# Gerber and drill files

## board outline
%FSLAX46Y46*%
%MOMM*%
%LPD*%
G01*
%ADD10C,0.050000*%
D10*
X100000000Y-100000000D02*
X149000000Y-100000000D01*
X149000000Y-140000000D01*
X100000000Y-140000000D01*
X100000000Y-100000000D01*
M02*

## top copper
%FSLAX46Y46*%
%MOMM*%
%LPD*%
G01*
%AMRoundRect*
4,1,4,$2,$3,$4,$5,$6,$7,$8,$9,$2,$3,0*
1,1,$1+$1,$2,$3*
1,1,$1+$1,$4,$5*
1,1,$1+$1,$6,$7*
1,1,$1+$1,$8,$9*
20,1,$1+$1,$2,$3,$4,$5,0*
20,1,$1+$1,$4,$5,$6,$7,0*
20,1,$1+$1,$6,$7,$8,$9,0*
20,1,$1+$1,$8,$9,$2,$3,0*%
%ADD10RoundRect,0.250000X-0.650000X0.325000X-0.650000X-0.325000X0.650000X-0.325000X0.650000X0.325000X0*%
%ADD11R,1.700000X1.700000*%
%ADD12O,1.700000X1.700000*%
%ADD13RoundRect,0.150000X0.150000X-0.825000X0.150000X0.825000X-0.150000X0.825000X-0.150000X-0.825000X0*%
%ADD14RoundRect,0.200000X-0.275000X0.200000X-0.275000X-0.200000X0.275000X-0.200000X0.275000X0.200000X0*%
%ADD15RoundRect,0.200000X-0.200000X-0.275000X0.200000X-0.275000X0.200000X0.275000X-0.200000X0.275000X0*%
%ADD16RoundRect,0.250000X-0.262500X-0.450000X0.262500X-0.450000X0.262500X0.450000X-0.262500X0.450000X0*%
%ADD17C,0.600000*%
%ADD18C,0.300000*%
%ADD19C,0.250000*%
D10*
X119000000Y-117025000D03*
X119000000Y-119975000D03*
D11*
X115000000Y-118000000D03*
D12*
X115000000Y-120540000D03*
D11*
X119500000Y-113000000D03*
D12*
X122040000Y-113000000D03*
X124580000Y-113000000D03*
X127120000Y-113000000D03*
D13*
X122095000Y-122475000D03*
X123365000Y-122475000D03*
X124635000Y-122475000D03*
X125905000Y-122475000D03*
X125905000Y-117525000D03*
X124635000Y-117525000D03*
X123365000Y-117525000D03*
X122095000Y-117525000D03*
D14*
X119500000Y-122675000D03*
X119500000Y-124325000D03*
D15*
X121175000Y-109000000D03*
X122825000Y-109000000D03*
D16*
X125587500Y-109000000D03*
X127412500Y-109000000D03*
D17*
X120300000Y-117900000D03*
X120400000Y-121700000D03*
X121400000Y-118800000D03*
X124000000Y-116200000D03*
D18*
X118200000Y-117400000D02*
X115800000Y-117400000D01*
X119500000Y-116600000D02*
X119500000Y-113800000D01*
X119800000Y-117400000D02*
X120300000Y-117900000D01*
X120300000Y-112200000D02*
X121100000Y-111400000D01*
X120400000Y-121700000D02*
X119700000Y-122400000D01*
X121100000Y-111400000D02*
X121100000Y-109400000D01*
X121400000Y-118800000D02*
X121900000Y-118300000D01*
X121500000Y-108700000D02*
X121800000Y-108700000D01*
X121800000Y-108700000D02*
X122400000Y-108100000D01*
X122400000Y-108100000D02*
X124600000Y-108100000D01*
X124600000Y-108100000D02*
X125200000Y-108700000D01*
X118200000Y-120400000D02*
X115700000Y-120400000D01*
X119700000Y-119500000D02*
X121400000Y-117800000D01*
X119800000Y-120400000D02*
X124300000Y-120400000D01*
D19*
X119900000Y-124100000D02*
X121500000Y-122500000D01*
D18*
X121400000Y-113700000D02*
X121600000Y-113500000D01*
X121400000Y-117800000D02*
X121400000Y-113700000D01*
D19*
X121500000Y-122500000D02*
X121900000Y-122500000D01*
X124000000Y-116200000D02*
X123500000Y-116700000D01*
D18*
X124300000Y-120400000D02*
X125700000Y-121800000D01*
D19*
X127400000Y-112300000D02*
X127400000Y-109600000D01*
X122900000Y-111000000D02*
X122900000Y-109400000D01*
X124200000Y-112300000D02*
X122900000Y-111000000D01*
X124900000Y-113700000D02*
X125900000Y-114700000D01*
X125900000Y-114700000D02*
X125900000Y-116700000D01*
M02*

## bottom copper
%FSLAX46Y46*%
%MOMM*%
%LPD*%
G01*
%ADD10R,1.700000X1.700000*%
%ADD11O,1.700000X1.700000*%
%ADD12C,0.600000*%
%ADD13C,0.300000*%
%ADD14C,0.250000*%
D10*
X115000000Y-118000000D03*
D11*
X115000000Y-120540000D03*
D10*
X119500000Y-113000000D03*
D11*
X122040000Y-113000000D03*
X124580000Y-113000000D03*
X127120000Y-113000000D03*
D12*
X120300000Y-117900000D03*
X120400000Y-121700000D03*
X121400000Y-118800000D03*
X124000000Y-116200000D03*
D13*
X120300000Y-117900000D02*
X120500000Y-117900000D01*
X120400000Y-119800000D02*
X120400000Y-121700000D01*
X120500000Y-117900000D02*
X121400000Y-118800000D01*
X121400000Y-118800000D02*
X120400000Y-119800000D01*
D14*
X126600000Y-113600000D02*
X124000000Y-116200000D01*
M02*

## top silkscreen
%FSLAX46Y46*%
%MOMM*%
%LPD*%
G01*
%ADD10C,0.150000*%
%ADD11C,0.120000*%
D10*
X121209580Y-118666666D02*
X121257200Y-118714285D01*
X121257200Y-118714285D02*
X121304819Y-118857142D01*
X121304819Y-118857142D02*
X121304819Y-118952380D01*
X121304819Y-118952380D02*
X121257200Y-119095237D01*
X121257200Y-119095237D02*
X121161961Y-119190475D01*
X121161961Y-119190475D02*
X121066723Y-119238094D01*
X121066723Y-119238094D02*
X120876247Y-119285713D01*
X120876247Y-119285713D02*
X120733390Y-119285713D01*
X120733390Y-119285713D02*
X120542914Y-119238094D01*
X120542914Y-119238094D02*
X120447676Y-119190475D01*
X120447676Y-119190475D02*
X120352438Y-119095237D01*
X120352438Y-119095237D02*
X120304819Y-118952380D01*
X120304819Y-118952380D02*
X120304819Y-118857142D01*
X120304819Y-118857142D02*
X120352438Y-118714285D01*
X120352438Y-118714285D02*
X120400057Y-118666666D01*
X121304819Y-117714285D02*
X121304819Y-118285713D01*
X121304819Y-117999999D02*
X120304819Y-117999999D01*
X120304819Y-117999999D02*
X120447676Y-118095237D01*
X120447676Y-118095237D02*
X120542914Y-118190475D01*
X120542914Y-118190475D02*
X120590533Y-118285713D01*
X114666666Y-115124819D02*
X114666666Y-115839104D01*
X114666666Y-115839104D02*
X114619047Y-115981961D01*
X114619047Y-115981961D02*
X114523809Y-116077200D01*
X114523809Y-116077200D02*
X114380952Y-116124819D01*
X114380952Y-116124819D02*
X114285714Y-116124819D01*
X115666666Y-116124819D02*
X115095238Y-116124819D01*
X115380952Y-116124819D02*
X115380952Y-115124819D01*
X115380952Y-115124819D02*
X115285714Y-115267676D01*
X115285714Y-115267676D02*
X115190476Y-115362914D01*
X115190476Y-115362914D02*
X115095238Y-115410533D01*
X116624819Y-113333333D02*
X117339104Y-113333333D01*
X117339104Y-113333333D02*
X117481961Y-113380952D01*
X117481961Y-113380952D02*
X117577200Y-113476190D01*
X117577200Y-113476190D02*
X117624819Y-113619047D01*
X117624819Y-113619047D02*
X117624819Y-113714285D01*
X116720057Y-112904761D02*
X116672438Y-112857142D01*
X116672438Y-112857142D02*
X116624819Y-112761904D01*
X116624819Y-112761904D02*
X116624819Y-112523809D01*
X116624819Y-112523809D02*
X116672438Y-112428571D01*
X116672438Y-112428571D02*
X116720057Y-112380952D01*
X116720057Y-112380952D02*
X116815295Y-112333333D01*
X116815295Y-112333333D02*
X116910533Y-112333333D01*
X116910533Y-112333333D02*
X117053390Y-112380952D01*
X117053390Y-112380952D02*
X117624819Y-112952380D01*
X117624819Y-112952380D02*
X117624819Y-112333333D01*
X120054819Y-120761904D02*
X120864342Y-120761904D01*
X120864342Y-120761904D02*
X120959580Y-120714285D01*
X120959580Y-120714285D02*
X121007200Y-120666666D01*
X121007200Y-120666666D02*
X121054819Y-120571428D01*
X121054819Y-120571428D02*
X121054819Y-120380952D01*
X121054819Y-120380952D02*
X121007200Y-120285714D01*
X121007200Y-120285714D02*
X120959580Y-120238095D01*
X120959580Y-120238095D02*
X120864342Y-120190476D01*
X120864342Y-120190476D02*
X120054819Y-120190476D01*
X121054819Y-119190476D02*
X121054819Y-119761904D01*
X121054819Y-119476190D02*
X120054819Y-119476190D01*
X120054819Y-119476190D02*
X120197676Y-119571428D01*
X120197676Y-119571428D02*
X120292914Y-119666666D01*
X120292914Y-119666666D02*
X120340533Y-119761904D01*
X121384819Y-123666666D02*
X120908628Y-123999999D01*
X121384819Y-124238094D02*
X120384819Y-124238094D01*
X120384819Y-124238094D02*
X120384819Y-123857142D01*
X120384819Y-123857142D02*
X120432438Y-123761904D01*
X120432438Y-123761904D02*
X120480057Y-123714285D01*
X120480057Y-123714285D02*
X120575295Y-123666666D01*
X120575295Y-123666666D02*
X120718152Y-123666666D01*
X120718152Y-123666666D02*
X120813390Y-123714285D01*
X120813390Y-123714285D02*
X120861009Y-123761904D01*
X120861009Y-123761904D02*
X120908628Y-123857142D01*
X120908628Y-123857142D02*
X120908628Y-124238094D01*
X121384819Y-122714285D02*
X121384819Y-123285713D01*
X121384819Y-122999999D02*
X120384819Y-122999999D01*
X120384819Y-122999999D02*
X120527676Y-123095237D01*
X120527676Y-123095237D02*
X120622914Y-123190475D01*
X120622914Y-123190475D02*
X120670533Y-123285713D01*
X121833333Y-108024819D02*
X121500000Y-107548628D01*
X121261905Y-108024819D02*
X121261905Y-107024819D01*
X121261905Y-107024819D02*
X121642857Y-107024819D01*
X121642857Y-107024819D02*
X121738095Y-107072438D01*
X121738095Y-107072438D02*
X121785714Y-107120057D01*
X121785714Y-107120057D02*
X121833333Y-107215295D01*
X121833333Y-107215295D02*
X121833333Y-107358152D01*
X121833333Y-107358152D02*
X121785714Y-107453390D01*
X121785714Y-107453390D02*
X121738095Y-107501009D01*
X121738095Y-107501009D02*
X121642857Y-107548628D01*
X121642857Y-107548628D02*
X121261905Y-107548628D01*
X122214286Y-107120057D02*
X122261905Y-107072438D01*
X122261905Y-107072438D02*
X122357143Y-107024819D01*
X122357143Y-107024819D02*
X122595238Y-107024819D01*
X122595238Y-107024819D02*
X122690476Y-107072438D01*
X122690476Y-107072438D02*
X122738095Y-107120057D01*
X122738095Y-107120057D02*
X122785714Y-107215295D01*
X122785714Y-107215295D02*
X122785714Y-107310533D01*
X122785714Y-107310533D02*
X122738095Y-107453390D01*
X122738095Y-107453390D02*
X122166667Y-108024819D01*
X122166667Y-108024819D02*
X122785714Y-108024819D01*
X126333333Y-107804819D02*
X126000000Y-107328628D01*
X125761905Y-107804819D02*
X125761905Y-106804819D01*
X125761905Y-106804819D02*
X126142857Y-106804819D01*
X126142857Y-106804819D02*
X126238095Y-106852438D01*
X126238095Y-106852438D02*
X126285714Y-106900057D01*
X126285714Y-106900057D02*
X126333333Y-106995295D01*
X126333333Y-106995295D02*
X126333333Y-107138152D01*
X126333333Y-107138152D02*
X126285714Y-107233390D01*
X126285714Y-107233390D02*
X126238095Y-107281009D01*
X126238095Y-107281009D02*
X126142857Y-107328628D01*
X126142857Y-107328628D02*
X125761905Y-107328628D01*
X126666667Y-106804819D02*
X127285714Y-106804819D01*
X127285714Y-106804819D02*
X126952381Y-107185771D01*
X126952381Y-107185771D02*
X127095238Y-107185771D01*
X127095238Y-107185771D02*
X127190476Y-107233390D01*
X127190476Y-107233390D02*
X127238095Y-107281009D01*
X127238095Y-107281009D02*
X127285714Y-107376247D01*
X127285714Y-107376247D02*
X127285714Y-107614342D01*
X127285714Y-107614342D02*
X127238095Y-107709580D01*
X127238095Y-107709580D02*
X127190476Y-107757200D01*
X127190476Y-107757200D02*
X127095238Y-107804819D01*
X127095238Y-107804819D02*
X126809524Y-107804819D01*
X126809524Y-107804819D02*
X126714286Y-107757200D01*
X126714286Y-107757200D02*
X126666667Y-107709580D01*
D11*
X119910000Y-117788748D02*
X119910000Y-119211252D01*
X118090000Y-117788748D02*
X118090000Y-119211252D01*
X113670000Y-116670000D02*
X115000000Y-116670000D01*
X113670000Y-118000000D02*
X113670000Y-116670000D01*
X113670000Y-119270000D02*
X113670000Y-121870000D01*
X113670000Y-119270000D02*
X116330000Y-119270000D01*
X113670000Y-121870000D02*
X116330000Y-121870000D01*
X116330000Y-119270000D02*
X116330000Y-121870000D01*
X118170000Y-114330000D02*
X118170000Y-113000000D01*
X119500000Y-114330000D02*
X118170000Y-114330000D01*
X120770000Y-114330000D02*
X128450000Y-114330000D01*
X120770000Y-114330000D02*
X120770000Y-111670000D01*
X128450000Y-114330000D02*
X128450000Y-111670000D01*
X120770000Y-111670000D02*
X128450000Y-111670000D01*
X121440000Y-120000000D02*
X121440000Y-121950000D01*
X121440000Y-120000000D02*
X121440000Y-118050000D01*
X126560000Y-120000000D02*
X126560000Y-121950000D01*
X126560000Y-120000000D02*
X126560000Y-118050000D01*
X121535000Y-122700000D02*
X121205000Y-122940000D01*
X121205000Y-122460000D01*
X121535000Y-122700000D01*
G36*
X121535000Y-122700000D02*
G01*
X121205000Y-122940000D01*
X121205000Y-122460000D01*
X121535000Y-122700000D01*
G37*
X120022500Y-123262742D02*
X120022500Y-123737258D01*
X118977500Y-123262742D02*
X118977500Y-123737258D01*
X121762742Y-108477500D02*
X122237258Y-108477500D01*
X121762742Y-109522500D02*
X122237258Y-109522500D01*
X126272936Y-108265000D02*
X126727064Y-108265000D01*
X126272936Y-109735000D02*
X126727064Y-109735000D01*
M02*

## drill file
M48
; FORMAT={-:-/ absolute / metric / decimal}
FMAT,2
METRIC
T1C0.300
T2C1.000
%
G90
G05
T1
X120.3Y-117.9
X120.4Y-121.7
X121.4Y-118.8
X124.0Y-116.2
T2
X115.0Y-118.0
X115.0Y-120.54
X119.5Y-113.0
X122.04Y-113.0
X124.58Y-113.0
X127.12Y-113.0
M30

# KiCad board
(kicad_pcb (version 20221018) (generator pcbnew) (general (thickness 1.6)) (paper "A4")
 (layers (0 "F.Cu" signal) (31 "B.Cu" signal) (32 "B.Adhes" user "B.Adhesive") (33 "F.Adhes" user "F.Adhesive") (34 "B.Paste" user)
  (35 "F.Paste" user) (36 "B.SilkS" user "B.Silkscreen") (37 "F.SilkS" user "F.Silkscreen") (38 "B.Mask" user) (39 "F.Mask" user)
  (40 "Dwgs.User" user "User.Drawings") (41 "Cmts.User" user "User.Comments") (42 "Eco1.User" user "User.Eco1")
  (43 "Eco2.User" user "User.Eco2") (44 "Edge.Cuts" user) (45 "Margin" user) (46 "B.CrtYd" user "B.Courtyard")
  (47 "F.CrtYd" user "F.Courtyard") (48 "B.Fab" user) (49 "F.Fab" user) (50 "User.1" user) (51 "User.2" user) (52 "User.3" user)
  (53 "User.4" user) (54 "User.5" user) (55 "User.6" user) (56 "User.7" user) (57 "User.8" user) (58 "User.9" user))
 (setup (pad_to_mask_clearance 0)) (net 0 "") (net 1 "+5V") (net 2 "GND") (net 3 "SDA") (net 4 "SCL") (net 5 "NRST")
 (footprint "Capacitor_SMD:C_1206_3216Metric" (layer "F.Cu") (at 119 118.5 -90)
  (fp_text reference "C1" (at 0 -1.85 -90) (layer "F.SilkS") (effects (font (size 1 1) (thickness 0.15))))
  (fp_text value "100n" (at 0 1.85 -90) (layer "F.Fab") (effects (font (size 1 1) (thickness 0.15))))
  (fp_line (start -0.711252 -0.91) (end 0.711252 -0.91) (stroke (width 0.12) (type solid)) (layer "F.SilkS"))
  (fp_line (start -0.711252 0.91) (end 0.711252 0.91) (stroke (width 0.12) (type solid)) (layer "F.SilkS"))
  (pad "1" smd roundrect (at -1.475 0 270) (size 1.15 1.8) (layers "F.Cu" "F.Paste" "F.Mask") (roundrect_rratio 0.217391) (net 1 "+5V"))
  (pad "2" smd roundrect (at 1.475 0 270) (size 1.15 1.8) (layers "F.Cu" "F.Paste" "F.Mask") (roundrect_rratio 0.217391) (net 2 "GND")))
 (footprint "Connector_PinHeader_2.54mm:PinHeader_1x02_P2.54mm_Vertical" (layer "F.Cu") (at 115 118)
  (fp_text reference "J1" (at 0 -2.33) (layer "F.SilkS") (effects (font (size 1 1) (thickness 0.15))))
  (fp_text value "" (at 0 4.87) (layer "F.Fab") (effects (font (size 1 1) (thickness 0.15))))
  (fp_line (start -1.33 -1.33) (end 0 -1.33) (stroke (width 0.12) (type solid)) (layer "F.SilkS"))
  (fp_line (start -1.33 0) (end -1.33 -1.33) (stroke (width 0.12) (type solid)) (layer "F.SilkS"))
  (fp_line (start -1.33 1.27) (end -1.33 3.87) (stroke (width 0.12) (type solid)) (layer "F.SilkS"))
  (fp_line (start -1.33 1.27) (end 1.33 1.27) (stroke (width 0.12) (type solid)) (layer "F.SilkS"))
  (fp_line (start -1.33 3.87) (end 1.33 3.87) (stroke (width 0.12) (type solid)) (layer "F.SilkS"))
  (fp_line (start 1.33 1.27) (end 1.33 3.87) (stroke (width 0.12) (type solid)) (layer "F.SilkS"))
  (pad "1" thru_hole rect (at 0 0) (size 1.7 1.7) (drill 1) (layers "*.Cu" "*.Mask") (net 1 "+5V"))
  (pad "2" thru_hole oval (at 0 2.54) (size 1.7 1.7) (drill 1) (layers "*.Cu" "*.Mask") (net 2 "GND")))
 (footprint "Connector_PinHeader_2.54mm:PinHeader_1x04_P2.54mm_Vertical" (layer "F.Cu") (at 119.5 113 90)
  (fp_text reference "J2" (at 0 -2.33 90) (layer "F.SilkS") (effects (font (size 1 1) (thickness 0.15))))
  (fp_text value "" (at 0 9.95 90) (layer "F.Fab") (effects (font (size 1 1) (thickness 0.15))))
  (fp_line (start -1.33 -1.33) (end 0 -1.33) (stroke (width 0.12) (type solid)) (layer "F.SilkS"))
  (fp_line (start -1.33 0) (end -1.33 -1.33) (stroke (width 0.12) (type solid)) (layer "F.SilkS"))
  (fp_line (start -1.33 1.27) (end -1.33 8.95) (stroke (width 0.12) (type solid)) (layer "F.SilkS"))
  (fp_line (start -1.33 1.27) (end 1.33 1.27) (stroke (width 0.12) (type solid)) (layer "F.SilkS"))
  (fp_line (start -1.33 8.95) (end 1.33 8.95) (stroke (width 0.12) (type solid)) (layer "F.SilkS"))
  (fp_line (start 1.33 1.27) (end 1.33 8.95) (stroke (width 0.12) (type solid)) (layer "F.SilkS"))
  (pad "1" thru_hole rect (at 0 0 90) (size 1.7 1.7) (drill 1) (layers "*.Cu" "*.Mask") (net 1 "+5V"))
  (pad "2" thru_hole oval (at 0 2.54 90) (size 1.7 1.7) (drill 1) (layers "*.Cu" "*.Mask") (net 2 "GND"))
  (pad "3" thru_hole oval (at 0 5.08 90) (size 1.7 1.7) (drill 1) (layers "*.Cu" "*.Mask") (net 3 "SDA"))
  (pad "4" thru_hole oval (at 0 7.62 90) (size 1.7 1.7) (drill 1) (layers "*.Cu" "*.Mask") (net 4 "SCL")))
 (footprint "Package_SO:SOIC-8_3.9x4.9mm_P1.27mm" (layer "F.Cu") (at 124 120 90)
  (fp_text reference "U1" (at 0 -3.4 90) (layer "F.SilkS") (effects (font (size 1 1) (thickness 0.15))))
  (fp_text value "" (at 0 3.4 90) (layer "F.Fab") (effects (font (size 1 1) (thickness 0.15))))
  (fp_line (start 0 -2.56) (end -1.95 -2.56) (stroke (width 0.12) (type solid)) (layer "F.SilkS"))
  (fp_line (start 0 -2.56) (end 1.95 -2.56) (stroke (width 0.12) (type solid)) (layer "F.SilkS"))
  (fp_line (start 0 2.56) (end -1.95 2.56) (stroke (width 0.12) (type solid)) (layer "F.SilkS"))
  (fp_line (start 0 2.56) (end 1.95 2.56) (stroke (width 0.12) (type solid)) (layer "F.SilkS"))
  (fp_poly
   (pts (xy -2.7 -2.465) (xy -2.94 -2.795) (xy -2.46 -2.795) (xy -2.7 -2.465)) (stroke (width 0.12) (type solid)) (fill solid)
   (layer "F.SilkS"))
  (pad "1" smd roundrect (at -2.475 -1.905 90) (size 1.95 0.6) (layers "F.Cu" "F.Paste" "F.Mask") (roundrect_rratio 0.25) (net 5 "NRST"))
  (pad "2" smd roundrect (at -2.475 -0.635 90) (size 1.95 0.6) (layers "F.Cu" "F.Paste" "F.Mask") (roundrect_rratio 0.25))
  (pad "3" smd roundrect (at -2.475 0.635 90) (size 1.95 0.6) (layers "F.Cu" "F.Paste" "F.Mask") (roundrect_rratio 0.25))
  (pad "4" smd roundrect (at -2.475 1.905 90) (size 1.95 0.6) (layers "F.Cu" "F.Paste" "F.Mask") (roundrect_rratio 0.25) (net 2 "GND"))
  (pad "5" smd roundrect (at 2.475 1.905 90) (size 1.95 0.6) (layers "F.Cu" "F.Paste" "F.Mask") (roundrect_rratio 0.25) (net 3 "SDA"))
  (pad "6" smd roundrect (at 2.475 0.635 90) (size 1.95 0.6) (layers "F.Cu" "F.Paste" "F.Mask") (roundrect_rratio 0.25))
  (pad "7" smd roundrect (at 2.475 -0.635 90) (size 1.95 0.6) (layers "F.Cu" "F.Paste" "F.Mask") (roundrect_rratio 0.25) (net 4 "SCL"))
  (pad "8" smd roundrect (at 2.475 -1.905 90) (size 1.95 0.6) (layers "F.Cu" "F.Paste" "F.Mask") (roundrect_rratio 0.25) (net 1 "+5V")))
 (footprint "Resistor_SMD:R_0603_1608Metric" (layer "F.Cu") (at 119.5 123.5 -90)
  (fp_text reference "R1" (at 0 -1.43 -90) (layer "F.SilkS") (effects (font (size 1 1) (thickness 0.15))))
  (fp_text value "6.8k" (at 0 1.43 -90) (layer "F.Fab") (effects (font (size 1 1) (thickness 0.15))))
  (fp_line (start -0.237258 -0.5225) (end 0.237258 -0.5225) (stroke (width 0.12) (type solid)) (layer "F.SilkS"))
  (fp_line (start -0.237258 0.5225) (end 0.237258 0.5225) (stroke (width 0.12) (type solid)) (layer "F.SilkS"))
  (pad "1" smd roundrect (at -0.825 0 270) (size 0.8 0.95) (layers "F.Cu" "F.Paste" "F.Mask") (roundrect_rratio 0.25) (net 1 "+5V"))
  (pad "2" smd roundrect (at 0.825 0 270) (size 0.8 0.95) (layers "F.Cu" "F.Paste" "F.Mask") (roundrect_rratio 0.25) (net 5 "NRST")))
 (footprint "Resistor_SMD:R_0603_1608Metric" (layer "F.Cu") (at 122 109)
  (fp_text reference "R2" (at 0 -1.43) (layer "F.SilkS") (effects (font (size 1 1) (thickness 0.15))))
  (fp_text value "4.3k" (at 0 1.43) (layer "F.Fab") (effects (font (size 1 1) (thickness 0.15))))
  (fp_line (start -0.237258 -0.5225) (end 0.237258 -0.5225) (stroke (width 0.12) (type solid)) (layer "F.SilkS"))
  (fp_line (start -0.237258 0.5225) (end 0.237258 0.5225) (stroke (width 0.12) (type solid)) (layer "F.SilkS"))
  (pad "1" smd roundrect (at -0.825 0) (size 0.8 0.95) (layers "F.Cu" "F.Paste" "F.Mask") (roundrect_rratio 0.25) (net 1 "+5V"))
  (pad "2" smd roundrect (at 0.825 0) (size 0.8 0.95) (layers "F.Cu" "F.Paste" "F.Mask") (roundrect_rratio 0.25) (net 3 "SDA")))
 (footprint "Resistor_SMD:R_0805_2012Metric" (layer "F.Cu") (at 126.5 109)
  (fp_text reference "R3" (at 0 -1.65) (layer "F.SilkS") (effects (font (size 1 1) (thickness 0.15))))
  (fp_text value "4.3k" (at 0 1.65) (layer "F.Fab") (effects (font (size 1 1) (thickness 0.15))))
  (fp_line (start -0.227064 -0.735) (end 0.227064 -0.735) (stroke (width 0.12) (type solid)) (layer "F.SilkS"))
  (fp_line (start -0.227064 0.735) (end 0.227064 0.735) (stroke (width 0.12) (type solid)) (layer "F.SilkS"))
  (pad "1" smd roundrect (at -0.9125 0) (size 1.025 1.4) (layers "F.Cu" "F.Paste" "F.Mask") (roundrect_rratio 0.243902) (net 1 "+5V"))
  (pad "2" smd roundrect (at 0.9125 0) (size 1.025 1.4) (layers "F.Cu" "F.Paste" "F.Mask") (roundrect_rratio 0.243902) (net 4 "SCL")))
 (gr_rect (start 100 100) (end 149 140) (stroke (width 0.05) (type default)) (fill none) (layer "Edge.Cuts"))
 (segment (start 118.2 117.4) (end 115.8 117.4) (width 0.3) (layer "F.Cu") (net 1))
 (segment (start 119.5 116.6) (end 119.5 113.8) (width 0.3) (layer "F.Cu") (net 1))
 (segment (start 119.8 117.4) (end 120.3 117.9) (width 0.3) (layer "F.Cu") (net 1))
 (segment (start 120.3 112.2) (end 121.1 111.4) (width 0.3) (layer "F.Cu") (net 1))
 (segment (start 120.4 121.7) (end 119.7 122.4) (width 0.3) (layer "F.Cu") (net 1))
 (segment (start 121.1 111.4) (end 121.1 109.4) (width 0.3) (layer "F.Cu") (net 1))
 (segment (start 121.4 118.8) (end 121.9 118.3) (width 0.3) (layer "F.Cu") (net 1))
 (segment (start 121.5 108.7) (end 121.8 108.7) (width 0.3) (layer "F.Cu") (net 1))
 (segment (start 121.8 108.7) (end 122.4 108.1) (width 0.3) (layer "F.Cu") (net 1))
 (segment (start 122.4 108.1) (end 124.6 108.1) (width 0.3) (layer "F.Cu") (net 1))
 (segment (start 124.6 108.1) (end 125.2 108.7) (width 0.3) (layer "F.Cu") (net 1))
 (via (at 120.3 117.9) (size 0.6) (drill 0.3) (layers "F.Cu" "B.Cu") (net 1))
 (via (at 120.4 121.7) (size 0.6) (drill 0.3) (layers "F.Cu" "B.Cu") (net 1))
 (via (at 121.4 118.8) (size 0.6) (drill 0.3) (layers "F.Cu" "B.Cu") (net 1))
 (segment (start 118.2 120.4) (end 115.7 120.4) (width 0.3) (layer "F.Cu") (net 2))
 (segment (start 119.7 119.5) (end 121.4 117.8) (width 0.3) (layer "F.Cu") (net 2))
 (segment (start 119.8 120.4) (end 124.3 120.4) (width 0.3) (layer "F.Cu") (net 2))
 (segment (start 119.9 124.1) (end 121.5 122.5) (width 0.25) (layer "F.Cu") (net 5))
 (segment (start 120.3 117.9) (end 120.5 117.9) (width 0.3) (layer "B.Cu") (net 1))
 (segment (start 120.4 119.8) (end 120.4 121.7) (width 0.3) (layer "B.Cu") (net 1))
 (segment (start 120.5 117.9) (end 121.4 118.8) (width 0.3) (layer "B.Cu") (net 1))
 (segment (start 121.4 113.7) (end 121.6 113.5) (width 0.3) (layer "F.Cu") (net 2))
 (segment (start 121.4 117.8) (end 121.4 113.7) (width 0.3) (layer "F.Cu") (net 2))
 (segment (start 121.4 118.8) (end 120.4 119.8) (width 0.3) (layer "B.Cu") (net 1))
 (segment (start 121.5 122.5) (end 121.9 122.5) (width 0.25) (layer "F.Cu") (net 5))
 (segment (start 124 116.2) (end 123.5 116.7) (width 0.25) (layer "F.Cu") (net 4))
 (segment (start 124.3 120.4) (end 125.7 121.8) (width 0.3) (layer "F.Cu") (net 2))
 (segment (start 127.4 112.3) (end 127.4 109.6) (width 0.25) (layer "F.Cu") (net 4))
 (via (at 124 116.2) (size 0.6) (drill 0.3) (layers "F.Cu" "B.Cu") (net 4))
 (segment (start 122.9 111) (end 122.9 109.4) (width 0.25) (layer "F.Cu") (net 3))
 (segment (start 124.2 112.3) (end 122.9 111) (width 0.25) (layer "F.Cu") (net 3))
 (segment (start 124.9 113.7) (end 125.9 114.7) (width 0.25) (layer "F.Cu") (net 3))
 (segment (start 125.9 114.7) (end 125.9 116.7) (width 0.25) (layer "F.Cu") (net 3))
 (segment (start 126.6 113.6) (end 124 116.2) (width 0.25) (layer "B.Cu") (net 4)))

